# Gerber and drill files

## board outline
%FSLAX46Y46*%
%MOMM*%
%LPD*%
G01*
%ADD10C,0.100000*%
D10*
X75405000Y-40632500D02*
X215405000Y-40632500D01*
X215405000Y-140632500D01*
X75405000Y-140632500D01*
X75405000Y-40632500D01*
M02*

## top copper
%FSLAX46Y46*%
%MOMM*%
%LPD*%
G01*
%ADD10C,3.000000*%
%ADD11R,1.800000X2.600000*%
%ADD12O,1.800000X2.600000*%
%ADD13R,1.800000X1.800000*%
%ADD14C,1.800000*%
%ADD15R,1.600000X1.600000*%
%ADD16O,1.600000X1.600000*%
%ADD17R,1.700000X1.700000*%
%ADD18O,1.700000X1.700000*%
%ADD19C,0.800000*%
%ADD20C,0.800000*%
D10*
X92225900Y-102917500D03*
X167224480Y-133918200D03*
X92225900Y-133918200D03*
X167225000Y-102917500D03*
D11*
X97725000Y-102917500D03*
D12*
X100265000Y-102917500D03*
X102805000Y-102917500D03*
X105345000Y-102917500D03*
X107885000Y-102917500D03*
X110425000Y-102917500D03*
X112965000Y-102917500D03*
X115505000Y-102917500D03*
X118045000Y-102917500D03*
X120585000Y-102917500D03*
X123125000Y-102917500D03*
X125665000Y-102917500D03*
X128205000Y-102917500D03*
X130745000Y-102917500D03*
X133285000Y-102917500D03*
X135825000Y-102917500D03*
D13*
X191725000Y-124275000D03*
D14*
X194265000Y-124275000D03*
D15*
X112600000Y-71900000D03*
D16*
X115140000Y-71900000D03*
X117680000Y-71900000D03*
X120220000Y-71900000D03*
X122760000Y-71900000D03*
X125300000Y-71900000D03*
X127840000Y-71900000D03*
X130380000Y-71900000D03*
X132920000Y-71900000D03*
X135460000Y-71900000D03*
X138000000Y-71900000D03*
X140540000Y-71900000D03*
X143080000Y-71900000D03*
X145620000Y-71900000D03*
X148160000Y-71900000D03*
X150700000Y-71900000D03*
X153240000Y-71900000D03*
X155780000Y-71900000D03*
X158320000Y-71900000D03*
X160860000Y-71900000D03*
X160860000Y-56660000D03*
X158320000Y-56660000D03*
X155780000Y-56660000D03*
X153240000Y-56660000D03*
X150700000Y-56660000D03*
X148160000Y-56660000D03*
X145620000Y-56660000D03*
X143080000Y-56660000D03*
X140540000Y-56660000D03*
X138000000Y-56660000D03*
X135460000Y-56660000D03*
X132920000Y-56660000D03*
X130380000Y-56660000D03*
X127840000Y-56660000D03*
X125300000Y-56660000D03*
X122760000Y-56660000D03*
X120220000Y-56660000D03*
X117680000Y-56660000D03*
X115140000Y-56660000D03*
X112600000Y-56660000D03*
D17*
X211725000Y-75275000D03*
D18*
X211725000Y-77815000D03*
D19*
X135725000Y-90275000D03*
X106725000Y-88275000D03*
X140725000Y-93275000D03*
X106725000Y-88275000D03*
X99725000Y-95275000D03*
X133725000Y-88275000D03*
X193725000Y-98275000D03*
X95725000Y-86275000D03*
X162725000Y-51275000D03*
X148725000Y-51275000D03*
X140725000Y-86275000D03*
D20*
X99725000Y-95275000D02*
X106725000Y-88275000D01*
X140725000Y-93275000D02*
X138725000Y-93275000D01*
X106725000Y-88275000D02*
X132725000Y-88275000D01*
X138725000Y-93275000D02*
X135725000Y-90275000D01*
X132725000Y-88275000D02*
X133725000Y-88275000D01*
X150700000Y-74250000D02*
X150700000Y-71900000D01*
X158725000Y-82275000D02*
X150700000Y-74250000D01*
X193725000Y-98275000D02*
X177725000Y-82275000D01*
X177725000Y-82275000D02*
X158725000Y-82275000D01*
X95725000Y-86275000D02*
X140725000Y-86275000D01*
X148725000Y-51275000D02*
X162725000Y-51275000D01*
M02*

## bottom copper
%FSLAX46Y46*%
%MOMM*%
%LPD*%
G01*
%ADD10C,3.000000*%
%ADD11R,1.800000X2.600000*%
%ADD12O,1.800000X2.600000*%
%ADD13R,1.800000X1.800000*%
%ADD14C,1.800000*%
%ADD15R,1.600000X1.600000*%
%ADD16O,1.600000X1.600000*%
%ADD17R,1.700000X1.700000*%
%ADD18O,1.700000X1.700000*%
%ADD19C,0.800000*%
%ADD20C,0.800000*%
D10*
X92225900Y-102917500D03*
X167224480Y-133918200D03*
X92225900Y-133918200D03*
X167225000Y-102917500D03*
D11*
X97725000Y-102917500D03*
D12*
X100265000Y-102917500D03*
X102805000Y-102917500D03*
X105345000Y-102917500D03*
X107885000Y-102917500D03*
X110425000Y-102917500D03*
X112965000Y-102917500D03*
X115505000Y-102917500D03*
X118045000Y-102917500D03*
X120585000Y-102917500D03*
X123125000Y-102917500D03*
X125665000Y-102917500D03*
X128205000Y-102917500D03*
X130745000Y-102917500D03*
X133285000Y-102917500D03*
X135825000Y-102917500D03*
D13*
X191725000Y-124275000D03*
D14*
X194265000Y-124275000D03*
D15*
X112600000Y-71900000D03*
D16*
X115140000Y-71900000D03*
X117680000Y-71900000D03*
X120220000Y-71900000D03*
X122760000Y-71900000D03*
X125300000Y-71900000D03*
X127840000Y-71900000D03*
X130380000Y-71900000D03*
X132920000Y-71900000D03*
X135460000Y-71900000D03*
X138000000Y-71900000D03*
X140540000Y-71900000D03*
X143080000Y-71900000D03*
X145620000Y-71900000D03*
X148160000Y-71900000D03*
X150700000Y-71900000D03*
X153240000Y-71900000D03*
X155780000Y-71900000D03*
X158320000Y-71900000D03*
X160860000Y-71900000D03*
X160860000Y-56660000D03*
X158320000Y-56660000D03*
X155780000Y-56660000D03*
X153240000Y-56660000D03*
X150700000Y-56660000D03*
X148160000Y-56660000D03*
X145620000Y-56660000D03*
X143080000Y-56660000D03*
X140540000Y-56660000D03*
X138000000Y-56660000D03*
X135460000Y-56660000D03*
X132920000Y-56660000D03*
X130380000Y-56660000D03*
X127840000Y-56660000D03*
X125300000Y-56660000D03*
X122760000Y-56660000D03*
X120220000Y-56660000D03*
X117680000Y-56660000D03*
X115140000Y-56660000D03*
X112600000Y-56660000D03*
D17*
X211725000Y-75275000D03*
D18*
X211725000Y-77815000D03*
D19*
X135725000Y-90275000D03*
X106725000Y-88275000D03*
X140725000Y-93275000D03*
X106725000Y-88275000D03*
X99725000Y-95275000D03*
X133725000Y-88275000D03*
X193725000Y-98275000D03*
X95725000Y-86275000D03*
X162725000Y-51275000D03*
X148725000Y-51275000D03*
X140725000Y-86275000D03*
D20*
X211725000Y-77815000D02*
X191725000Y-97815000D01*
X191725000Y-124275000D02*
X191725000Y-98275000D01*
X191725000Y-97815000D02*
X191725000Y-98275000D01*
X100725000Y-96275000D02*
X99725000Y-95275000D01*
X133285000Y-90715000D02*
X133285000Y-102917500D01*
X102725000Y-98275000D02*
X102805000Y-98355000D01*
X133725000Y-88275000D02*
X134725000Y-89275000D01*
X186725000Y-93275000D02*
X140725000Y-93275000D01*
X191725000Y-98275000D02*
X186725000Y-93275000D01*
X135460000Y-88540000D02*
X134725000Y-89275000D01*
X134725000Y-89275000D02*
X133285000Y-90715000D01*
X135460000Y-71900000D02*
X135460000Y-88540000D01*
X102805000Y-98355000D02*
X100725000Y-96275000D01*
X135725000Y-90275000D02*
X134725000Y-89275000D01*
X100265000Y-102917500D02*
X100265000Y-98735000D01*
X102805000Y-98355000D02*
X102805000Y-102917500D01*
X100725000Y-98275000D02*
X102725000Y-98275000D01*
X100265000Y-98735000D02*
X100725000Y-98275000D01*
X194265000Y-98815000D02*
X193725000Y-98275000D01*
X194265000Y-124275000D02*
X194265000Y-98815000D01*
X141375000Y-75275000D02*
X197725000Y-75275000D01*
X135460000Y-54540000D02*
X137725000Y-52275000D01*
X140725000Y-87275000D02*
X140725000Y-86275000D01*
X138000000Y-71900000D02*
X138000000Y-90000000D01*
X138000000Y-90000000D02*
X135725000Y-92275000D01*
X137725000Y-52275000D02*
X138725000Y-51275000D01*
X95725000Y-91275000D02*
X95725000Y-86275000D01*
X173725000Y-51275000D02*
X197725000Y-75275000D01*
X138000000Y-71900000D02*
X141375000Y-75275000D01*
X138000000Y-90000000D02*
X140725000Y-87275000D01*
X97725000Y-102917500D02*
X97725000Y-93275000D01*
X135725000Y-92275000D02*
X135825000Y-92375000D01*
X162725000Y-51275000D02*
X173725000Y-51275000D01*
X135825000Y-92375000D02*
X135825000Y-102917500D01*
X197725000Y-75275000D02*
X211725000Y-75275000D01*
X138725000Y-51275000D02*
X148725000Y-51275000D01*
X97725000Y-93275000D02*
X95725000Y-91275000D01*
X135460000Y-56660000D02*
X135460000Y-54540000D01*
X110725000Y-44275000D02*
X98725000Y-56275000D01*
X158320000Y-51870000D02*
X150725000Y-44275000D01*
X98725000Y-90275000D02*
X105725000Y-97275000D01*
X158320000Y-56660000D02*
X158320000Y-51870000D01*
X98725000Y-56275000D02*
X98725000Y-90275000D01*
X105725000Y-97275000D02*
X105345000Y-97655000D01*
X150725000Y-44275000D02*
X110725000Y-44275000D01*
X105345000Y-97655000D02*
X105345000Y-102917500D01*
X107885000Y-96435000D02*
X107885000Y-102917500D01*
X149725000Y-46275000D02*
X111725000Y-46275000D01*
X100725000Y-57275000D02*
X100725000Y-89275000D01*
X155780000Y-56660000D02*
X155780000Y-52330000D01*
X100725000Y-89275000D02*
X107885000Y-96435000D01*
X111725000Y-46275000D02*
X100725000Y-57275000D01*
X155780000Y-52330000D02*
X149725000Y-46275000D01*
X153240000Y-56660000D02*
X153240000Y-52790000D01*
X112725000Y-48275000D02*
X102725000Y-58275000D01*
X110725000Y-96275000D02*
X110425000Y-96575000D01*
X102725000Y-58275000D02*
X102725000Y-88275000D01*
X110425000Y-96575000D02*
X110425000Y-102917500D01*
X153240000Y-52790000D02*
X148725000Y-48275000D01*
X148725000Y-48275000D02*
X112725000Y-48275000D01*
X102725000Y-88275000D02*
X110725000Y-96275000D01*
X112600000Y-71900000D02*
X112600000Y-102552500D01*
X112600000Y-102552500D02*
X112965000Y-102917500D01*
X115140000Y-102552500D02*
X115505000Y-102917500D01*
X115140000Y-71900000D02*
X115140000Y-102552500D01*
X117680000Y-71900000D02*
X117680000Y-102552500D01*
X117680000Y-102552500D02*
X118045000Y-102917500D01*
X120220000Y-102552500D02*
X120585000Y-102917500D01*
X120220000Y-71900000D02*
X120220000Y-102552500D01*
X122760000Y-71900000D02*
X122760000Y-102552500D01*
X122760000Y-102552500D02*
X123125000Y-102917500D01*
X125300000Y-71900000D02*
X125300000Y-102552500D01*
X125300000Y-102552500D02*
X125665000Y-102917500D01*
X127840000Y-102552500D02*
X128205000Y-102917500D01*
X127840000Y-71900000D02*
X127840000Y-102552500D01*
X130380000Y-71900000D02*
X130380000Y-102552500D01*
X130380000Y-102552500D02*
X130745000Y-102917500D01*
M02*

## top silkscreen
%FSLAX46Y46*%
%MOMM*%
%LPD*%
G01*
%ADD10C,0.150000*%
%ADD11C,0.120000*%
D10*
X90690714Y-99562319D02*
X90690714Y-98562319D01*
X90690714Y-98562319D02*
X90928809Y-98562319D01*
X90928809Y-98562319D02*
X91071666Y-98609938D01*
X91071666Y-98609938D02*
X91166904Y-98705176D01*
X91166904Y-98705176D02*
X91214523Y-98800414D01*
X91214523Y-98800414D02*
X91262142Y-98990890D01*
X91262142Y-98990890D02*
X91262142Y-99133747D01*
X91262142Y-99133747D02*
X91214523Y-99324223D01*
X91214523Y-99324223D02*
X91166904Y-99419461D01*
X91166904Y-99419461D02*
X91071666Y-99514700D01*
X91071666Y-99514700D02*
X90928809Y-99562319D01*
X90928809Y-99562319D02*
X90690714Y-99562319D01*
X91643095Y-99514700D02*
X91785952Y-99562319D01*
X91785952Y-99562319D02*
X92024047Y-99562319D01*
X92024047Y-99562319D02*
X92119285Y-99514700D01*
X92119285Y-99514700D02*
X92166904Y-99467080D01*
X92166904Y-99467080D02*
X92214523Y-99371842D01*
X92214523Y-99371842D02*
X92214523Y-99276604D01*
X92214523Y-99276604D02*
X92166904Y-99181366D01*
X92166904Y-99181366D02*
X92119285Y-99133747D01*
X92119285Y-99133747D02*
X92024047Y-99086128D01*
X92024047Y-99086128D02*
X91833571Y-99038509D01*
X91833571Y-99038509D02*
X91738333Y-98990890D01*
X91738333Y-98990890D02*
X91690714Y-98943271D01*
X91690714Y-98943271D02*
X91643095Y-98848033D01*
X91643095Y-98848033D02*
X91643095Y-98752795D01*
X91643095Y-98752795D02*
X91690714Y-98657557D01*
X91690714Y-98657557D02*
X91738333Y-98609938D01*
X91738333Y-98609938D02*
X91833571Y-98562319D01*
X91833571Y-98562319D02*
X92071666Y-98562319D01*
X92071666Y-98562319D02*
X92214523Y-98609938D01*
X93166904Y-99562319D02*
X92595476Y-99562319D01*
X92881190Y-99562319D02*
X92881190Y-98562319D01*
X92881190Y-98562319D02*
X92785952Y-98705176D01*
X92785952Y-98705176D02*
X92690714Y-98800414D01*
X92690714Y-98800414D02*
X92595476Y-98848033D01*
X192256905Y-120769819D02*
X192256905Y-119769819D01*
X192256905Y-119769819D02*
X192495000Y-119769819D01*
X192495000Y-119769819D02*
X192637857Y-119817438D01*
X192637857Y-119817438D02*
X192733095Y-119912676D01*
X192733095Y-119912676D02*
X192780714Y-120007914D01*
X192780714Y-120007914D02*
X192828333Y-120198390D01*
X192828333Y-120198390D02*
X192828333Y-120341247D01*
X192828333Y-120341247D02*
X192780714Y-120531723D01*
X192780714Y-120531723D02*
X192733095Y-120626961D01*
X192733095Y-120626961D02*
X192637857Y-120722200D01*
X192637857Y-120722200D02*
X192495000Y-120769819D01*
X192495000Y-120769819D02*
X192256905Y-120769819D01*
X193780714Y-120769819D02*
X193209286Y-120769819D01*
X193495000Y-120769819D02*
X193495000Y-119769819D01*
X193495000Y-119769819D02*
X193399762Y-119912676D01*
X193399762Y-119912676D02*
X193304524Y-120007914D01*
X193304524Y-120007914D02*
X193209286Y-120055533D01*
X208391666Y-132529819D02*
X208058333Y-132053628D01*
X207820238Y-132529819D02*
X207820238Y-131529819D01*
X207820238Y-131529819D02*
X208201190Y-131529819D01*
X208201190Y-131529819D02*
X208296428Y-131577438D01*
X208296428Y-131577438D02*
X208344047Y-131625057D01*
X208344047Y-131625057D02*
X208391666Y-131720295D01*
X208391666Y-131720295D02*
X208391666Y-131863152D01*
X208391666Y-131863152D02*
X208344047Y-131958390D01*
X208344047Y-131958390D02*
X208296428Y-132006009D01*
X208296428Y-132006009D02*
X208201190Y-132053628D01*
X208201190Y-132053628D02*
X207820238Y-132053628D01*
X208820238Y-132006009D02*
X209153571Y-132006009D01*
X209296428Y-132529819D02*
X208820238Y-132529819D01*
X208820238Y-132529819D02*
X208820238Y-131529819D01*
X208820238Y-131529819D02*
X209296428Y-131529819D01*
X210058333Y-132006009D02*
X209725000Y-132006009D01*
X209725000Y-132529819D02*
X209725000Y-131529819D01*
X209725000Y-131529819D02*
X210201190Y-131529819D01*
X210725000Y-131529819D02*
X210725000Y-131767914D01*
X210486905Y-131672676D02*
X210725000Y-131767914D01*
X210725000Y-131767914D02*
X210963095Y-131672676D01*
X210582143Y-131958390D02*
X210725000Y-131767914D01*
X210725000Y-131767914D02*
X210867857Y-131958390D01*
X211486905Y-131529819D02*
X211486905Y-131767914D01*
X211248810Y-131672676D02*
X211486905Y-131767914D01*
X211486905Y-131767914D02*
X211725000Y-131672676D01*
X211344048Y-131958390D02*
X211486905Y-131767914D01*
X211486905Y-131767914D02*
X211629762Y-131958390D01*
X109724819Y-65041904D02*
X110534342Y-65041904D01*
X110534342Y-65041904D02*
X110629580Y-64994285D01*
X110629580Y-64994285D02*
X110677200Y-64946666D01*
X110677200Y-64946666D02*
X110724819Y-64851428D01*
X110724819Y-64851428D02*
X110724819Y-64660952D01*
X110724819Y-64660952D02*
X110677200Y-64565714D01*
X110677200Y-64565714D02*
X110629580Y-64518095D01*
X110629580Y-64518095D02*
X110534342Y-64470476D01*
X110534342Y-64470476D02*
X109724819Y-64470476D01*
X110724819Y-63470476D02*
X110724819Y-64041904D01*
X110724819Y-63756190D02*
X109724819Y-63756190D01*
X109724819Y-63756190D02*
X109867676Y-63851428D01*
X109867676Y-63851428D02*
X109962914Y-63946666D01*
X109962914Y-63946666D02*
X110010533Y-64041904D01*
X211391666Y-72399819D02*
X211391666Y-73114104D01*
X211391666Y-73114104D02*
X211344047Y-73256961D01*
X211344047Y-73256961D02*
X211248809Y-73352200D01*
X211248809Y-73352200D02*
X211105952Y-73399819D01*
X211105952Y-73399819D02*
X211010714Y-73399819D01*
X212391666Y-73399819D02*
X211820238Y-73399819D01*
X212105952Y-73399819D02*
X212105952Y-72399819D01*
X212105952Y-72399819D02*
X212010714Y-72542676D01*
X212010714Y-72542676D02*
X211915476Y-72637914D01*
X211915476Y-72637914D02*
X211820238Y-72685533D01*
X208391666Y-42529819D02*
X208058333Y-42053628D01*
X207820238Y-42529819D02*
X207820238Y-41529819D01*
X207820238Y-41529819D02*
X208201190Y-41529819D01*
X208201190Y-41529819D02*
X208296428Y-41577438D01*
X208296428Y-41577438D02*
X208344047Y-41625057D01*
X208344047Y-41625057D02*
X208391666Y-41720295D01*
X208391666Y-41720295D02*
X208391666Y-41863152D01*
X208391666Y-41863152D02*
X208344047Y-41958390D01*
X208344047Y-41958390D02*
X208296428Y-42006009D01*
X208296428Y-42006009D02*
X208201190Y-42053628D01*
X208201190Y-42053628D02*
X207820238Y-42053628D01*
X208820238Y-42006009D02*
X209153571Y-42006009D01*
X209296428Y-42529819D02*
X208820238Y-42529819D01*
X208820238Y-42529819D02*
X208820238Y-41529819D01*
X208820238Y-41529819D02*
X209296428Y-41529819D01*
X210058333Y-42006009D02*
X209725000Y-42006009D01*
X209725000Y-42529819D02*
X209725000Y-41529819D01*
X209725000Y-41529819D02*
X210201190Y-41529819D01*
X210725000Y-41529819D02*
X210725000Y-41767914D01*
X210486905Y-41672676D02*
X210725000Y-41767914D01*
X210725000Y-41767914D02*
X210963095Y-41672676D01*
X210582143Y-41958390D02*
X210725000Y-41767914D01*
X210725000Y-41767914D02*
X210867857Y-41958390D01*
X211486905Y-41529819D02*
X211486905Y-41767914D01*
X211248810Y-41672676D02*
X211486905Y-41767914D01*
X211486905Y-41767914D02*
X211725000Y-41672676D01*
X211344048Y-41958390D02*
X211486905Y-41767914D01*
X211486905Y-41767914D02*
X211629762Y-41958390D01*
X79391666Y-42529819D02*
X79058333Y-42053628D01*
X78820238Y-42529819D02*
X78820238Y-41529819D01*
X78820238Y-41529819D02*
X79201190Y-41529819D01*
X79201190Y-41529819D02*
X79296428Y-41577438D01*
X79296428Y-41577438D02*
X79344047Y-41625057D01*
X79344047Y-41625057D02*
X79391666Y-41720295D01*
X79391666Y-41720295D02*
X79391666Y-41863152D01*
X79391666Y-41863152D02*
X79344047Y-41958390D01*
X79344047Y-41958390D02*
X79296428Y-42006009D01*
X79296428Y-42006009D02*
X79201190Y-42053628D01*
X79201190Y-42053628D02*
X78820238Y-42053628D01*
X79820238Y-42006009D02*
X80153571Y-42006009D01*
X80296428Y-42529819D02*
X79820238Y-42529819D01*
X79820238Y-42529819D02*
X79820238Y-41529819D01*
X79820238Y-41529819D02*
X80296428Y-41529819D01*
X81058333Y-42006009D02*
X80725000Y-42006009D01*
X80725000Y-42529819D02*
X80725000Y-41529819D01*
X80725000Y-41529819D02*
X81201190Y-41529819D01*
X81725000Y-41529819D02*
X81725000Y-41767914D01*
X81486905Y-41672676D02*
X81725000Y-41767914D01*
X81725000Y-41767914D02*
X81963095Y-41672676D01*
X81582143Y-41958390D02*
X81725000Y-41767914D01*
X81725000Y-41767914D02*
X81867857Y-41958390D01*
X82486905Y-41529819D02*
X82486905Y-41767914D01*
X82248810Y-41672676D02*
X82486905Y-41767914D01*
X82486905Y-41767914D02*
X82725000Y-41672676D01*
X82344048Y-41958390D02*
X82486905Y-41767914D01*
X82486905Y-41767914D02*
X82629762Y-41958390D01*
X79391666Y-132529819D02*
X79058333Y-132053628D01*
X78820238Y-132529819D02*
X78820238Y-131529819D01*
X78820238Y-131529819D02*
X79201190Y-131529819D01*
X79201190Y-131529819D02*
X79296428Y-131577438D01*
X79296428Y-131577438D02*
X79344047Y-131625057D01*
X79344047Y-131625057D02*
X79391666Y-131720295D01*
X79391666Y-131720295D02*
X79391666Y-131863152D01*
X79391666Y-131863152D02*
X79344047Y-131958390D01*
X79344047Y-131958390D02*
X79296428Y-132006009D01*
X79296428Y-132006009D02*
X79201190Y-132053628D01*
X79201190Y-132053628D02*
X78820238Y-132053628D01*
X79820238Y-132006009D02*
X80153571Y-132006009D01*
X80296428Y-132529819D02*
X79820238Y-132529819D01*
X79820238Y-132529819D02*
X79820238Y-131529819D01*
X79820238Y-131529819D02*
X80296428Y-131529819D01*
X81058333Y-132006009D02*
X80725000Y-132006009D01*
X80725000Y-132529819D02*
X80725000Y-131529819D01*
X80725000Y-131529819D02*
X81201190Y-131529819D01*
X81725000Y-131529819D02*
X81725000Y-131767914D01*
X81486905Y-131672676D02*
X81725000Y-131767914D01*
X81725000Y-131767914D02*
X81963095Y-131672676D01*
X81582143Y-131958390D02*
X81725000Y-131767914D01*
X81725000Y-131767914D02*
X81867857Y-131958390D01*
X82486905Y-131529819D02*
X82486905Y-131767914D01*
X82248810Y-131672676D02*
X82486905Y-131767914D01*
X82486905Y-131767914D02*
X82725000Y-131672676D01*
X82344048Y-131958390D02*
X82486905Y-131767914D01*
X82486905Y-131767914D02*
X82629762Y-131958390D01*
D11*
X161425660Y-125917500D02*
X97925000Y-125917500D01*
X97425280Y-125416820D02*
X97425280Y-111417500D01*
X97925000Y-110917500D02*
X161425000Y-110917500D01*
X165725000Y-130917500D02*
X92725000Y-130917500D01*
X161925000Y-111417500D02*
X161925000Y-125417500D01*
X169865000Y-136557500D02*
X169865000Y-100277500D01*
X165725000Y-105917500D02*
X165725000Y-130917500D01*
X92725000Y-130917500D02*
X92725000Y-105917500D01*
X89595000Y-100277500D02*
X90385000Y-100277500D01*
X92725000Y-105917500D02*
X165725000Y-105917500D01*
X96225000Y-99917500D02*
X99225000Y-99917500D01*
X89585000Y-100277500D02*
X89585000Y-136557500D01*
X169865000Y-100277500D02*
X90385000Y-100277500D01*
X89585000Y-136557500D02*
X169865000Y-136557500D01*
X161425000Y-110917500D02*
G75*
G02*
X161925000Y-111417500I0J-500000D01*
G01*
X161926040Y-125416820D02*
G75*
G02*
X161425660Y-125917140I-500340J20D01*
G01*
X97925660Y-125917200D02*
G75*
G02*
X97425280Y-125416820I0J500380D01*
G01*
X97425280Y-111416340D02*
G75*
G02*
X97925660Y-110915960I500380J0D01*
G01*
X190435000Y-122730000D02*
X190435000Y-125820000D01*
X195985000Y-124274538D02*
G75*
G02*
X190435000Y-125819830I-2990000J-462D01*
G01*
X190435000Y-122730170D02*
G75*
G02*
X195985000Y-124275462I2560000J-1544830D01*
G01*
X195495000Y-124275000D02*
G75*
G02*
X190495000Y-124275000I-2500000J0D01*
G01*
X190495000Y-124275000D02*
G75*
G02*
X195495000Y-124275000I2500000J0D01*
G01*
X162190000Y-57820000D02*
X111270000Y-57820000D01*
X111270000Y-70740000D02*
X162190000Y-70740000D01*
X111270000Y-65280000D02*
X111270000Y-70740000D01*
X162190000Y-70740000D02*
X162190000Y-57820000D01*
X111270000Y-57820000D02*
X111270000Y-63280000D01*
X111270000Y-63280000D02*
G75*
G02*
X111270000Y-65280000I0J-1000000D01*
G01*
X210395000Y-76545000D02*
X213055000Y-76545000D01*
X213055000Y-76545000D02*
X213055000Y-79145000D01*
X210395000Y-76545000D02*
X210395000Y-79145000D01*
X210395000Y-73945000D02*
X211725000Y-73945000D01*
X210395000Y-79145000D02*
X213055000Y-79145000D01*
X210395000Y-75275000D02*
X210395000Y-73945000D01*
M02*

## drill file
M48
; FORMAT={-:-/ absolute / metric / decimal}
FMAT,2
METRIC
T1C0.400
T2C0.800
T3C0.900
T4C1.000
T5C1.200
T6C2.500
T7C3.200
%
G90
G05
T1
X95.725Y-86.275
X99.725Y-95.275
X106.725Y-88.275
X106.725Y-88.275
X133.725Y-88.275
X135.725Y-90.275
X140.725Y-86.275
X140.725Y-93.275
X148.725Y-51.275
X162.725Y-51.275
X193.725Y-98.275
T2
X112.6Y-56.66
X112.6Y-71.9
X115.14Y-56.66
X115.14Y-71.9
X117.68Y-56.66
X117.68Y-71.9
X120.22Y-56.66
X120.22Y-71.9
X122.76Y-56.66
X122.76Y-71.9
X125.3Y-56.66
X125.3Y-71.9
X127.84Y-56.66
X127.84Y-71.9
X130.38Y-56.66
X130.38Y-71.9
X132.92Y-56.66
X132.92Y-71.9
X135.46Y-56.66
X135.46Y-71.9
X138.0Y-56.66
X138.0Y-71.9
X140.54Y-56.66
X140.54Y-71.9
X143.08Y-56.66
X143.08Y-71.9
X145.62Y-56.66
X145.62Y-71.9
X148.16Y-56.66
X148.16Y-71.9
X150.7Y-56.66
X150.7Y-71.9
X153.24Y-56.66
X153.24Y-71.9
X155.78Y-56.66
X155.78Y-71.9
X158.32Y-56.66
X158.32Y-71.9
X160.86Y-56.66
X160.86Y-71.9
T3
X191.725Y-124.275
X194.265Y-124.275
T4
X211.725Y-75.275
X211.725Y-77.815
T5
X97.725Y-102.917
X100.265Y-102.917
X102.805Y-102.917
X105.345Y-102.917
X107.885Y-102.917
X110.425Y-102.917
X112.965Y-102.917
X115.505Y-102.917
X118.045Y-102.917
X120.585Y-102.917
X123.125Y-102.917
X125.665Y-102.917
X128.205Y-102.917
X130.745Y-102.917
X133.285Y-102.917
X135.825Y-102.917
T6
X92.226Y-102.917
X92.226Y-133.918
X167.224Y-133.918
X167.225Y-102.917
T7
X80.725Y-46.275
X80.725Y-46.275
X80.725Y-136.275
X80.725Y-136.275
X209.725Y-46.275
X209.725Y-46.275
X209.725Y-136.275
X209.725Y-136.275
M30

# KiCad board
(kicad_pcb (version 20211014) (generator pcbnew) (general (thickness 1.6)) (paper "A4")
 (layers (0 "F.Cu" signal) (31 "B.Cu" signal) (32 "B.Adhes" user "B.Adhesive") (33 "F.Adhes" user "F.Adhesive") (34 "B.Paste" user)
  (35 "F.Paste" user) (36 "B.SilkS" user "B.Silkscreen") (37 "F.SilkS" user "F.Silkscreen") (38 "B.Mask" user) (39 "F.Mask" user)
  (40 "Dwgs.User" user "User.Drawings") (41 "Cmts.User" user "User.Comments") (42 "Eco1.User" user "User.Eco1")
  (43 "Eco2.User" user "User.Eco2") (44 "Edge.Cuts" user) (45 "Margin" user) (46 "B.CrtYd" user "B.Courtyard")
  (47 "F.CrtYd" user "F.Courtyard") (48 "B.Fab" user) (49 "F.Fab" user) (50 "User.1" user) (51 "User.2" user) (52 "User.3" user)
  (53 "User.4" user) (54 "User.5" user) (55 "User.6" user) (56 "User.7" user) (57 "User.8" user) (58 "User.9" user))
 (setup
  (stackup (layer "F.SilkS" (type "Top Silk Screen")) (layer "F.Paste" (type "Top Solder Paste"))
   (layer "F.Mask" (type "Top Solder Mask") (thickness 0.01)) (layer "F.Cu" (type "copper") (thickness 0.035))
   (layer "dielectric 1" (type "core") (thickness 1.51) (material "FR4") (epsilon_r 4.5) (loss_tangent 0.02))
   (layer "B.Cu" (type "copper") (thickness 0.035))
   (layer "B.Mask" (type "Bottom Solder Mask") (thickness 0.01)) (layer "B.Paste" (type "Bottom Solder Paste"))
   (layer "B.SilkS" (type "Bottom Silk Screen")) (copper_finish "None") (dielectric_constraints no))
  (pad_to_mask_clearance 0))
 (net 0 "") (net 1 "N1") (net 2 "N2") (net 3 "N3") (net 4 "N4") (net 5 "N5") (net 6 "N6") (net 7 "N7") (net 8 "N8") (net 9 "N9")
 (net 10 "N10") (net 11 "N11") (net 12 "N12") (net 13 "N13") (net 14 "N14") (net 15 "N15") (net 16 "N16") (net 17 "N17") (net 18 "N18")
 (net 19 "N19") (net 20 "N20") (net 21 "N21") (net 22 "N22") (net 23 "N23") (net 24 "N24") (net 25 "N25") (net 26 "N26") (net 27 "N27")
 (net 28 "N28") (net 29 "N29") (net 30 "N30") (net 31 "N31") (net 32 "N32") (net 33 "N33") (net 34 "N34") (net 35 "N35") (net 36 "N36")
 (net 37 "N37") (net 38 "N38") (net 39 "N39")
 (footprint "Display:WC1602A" (layer "F.Cu") (at 97.725 102.9175)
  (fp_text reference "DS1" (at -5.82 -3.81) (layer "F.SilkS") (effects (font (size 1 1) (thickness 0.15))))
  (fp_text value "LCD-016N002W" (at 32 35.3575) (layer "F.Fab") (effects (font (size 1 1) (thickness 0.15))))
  (fp_line (start 63.70066 23) (end 0.2 23) (layer "F.SilkS") (width 0.12))
  (fp_line (start -0.29972 22.49932) (end -0.29972 8.5) (layer "F.SilkS") (width 0.12))
  (fp_line (start 0.2 8) (end 63.7 8) (layer "F.SilkS") (width 0.12))
  (fp_line (start 68 28) (end -5 28) (layer "F.SilkS") (width 0.12))
  (fp_line (start 64.2 8.5) (end 64.2 22.5) (layer "F.SilkS") (width 0.12))
  (fp_line (start 72.14 33.64) (end 72.14 -2.64) (layer "F.SilkS") (width 0.12))
  (fp_line (start 68 3) (end 68 28) (layer "F.SilkS") (width 0.12))
  (fp_line (start -5 28) (end -5 3) (layer "F.SilkS") (width 0.12))
  (fp_line (start -8.13 -2.64) (end -7.34 -2.64) (layer "F.SilkS") (width 0.12))
  (fp_line (start -5 3) (end 68 3) (layer "F.SilkS") (width 0.12))
  (fp_line (start -1.5 -3) (end 1.5 -3) (layer "F.SilkS") (width 0.12))
  (fp_line (start -8.14 -2.64) (end -8.14 33.64) (layer "F.SilkS") (width 0.12))
  (fp_line (start 72.14 -2.64) (end -7.34 -2.64) (layer "F.SilkS") (width 0.12))
  (fp_line (start -8.14 33.64) (end 72.14 33.64) (layer "F.SilkS") (width 0.12))
  (fp_arc (start 63.7 8) (mid 64.053553 8.146447) (end 64.2 8.5) (layer "F.SilkS") (width 0.12))
  (fp_arc (start 64.20104 22.49932) (mid 64.054479 22.85315) (end 63.70066 22.9997) (layer "F.SilkS") (width 0.12))
  (fp_arc (start 0.20066 22.9997) (mid -0.153162 22.853142) (end -0.29972 22.49932) (layer "F.SilkS") (width 0.12))
  (fp_arc (start -0.29972 8.49884) (mid -0.153162 8.145018) (end 0.20066 7.99846) (layer "F.SilkS") (width 0.12))
  (pad "" thru_hole circle (at -5.4991 0) (size 3 3) (drill 2.5) (layers *.Cu *.Mask))
  (pad "" thru_hole circle (at 69.49948 31.0007) (size 3 3) (drill 2.5) (layers *.Cu *.Mask))
  (pad "" thru_hole circle (at -5.4991 31.0007) (size 3 3) (drill 2.5) (layers *.Cu *.Mask))
  (pad "" thru_hole circle (at 69.5 0) (size 3 3) (drill 2.5) (layers *.Cu *.Mask))
  (pad "1" thru_hole rect (at 0 0) (size 1.8 2.6) (drill 1.2) (layers *.Cu *.Mask) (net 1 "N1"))
  (pad "2" thru_hole oval (at 2.54 0) (size 1.8 2.6) (drill 1.2) (layers *.Cu *.Mask) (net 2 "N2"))
  (pad "3" thru_hole oval (at 5.08 0) (size 1.8 2.6) (drill 1.2) (layers *.Cu *.Mask) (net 2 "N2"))
  (pad "4" thru_hole oval (at 7.62 0) (size 1.8 2.6) (drill 1.2) (layers *.Cu *.Mask) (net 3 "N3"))
  (pad "5" thru_hole oval (at 10.16 0) (size 1.8 2.6) (drill 1.2) (layers *.Cu *.Mask) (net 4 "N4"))
  (pad "6" thru_hole oval (at 12.7 0) (size 1.8 2.6) (drill 1.2) (layers *.Cu *.Mask) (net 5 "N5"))
  (pad "7" thru_hole oval (at 15.24 0) (size 1.8 2.6) (drill 1.2) (layers *.Cu *.Mask) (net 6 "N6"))
  (pad "8" thru_hole oval (at 17.78 0) (size 1.8 2.6) (drill 1.2) (layers *.Cu *.Mask) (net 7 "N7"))
  (pad "9" thru_hole oval (at 20.32 0) (size 1.8 2.6) (drill 1.2) (layers *.Cu *.Mask) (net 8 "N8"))
  (pad "10" thru_hole oval (at 22.86 0) (size 1.8 2.6) (drill 1.2) (layers *.Cu *.Mask) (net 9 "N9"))
  (pad "11" thru_hole oval (at 25.4 0) (size 1.8 2.6) (drill 1.2) (layers *.Cu *.Mask) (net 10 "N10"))
  (pad "12" thru_hole oval (at 27.94 0) (size 1.8 2.6) (drill 1.2) (layers *.Cu *.Mask) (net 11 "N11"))
  (pad "13" thru_hole oval (at 30.48 0) (size 1.8 2.6) (drill 1.2) (layers *.Cu *.Mask) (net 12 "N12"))
  (pad "14" thru_hole oval (at 33.02 0) (size 1.8 2.6) (drill 1.2) (layers *.Cu *.Mask) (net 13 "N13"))
  (pad "15" thru_hole oval (at 35.56 0) (size 1.8 2.6) (drill 1.2) (layers *.Cu *.Mask) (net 2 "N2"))
  (pad "16" thru_hole oval (at 38.1 0) (size 1.8 2.6) (drill 1.2) (layers *.Cu *.Mask) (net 1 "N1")))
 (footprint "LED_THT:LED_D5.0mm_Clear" (layer "F.Cu") (at 191.725 124.275)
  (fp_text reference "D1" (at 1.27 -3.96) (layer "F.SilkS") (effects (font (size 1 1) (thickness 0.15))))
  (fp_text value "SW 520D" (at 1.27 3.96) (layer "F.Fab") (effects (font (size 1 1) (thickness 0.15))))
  (fp_line (start -1.29 -1.545) (end -1.29 1.545) (layer "F.SilkS") (width 0.12))
  (fp_arc (start 4.26 -0.000462) (mid 2.072002 2.880433) (end -1.29 1.54483) (layer "F.SilkS") (width 0.12))
  (fp_arc (start -1.29 -1.54483) (mid 2.072002 -2.880433) (end 4.26 0.000462) (layer "F.SilkS") (width 0.12))
  (fp_circle (center 1.27 0) (end 3.77 0) (layer "F.SilkS") (width 0.12) (fill none))
  (pad "1" thru_hole rect (at 0 0) (size 1.8 1.8) (drill 0.9) (layers *.Cu *.Mask) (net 2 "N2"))
  (pad "2" thru_hole circle (at 2.54 0) (size 1.8 1.8) (drill 0.9) (layers *.Cu *.Mask) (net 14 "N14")))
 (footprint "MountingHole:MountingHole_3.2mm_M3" (layer "F.Cu") (at 209.725 136.275)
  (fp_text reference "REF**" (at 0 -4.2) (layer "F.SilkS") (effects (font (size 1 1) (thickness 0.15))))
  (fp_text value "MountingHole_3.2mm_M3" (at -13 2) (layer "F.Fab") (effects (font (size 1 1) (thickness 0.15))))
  (pad "" np_thru_hole circle (at 0 0) (size 3.2 3.2) (drill 3.2) (layers *.Cu *.Mask))
  (pad "" np_thru_hole circle (at 0 0) (size 3.2 3.2) (drill 3.2) (layers *.Cu *.Mask)))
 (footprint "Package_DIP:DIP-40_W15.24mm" (layer "F.Cu") (at 112.6 71.9 90)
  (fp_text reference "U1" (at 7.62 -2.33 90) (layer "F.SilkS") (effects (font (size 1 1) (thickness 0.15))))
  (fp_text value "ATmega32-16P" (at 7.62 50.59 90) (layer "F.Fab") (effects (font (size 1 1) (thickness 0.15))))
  (fp_line (start 14.08 49.59) (end 14.08 -1.33) (layer "F.SilkS") (width 0.12))
  (fp_line (start 1.16 -1.33) (end 1.16 49.59) (layer "F.SilkS") (width 0.12))
  (fp_line (start 6.62 -1.33) (end 1.16 -1.33) (layer "F.SilkS") (width 0.12))
  (fp_line (start 1.16 49.59) (end 14.08 49.59) (layer "F.SilkS") (width 0.12))
  (fp_line (start 14.08 -1.33) (end 8.62 -1.33) (layer "F.SilkS") (width 0.12))
  (fp_arc (start 8.62 -1.33) (mid 7.62 -0.33) (end 6.62 -1.33) (layer "F.SilkS") (width 0.12))
  (pad "1" thru_hole rect (at 0 0 90) (size 1.6 1.6) (drill 0.8) (layers *.Cu *.Mask) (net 6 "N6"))
  (pad "2" thru_hole oval (at 0 2.54 90) (size 1.6 1.6) (drill 0.8) (layers *.Cu *.Mask) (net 7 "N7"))
  (pad "3" thru_hole oval (at 0 5.08 90) (size 1.6 1.6) (drill 0.8) (layers *.Cu *.Mask) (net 8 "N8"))
  (pad "4" thru_hole oval (at 0 7.62 90) (size 1.6 1.6) (drill 0.8) (layers *.Cu *.Mask) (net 9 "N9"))
  (pad "5" thru_hole oval (at 0 10.16 90) (size 1.6 1.6) (drill 0.8) (layers *.Cu *.Mask) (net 10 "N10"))
  (pad "6" thru_hole oval (at 0 12.7 90) (size 1.6 1.6) (drill 0.8) (layers *.Cu *.Mask) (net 11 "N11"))
  (pad "7" thru_hole oval (at 0 15.24 90) (size 1.6 1.6) (drill 0.8) (layers *.Cu *.Mask) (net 12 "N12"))
  (pad "8" thru_hole oval (at 0 17.78 90) (size 1.6 1.6) (drill 0.8) (layers *.Cu *.Mask) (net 13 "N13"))
  (pad "9" thru_hole oval (at 0 20.32 90) (size 1.6 1.6) (drill 0.8) (layers *.Cu *.Mask) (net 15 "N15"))
  (pad "10" thru_hole oval (at 0 22.86 90) (size 1.6 1.6) (drill 0.8) (layers *.Cu *.Mask) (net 2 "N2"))
  (pad "11" thru_hole oval (at 0 25.4 90) (size 1.6 1.6) (drill 0.8) (layers *.Cu *.Mask) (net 1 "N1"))
  (pad "12" thru_hole oval (at 0 27.94 90) (size 1.6 1.6) (drill 0.8) (layers *.Cu *.Mask) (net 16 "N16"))
  (pad "13" thru_hole oval (at 0 30.48 90) (size 1.6 1.6) (drill 0.8) (layers *.Cu *.Mask) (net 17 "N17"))
  (pad "14" thru_hole oval (at 0 33.02 90) (size 1.6 1.6) (drill 0.8) (layers *.Cu *.Mask) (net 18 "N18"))
  (pad "15" thru_hole oval (at 0 35.56 90) (size 1.6 1.6) (drill 0.8) (layers *.Cu *.Mask) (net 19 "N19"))
  (pad "16" thru_hole oval (at 0 38.1 90) (size 1.6 1.6) (drill 0.8) (layers *.Cu *.Mask) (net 14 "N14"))
  (pad "17" thru_hole oval (at 0 40.64 90) (size 1.6 1.6) (drill 0.8) (layers *.Cu *.Mask) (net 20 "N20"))
  (pad "18" thru_hole oval (at 0 43.18 90) (size 1.6 1.6) (drill 0.8) (layers *.Cu *.Mask) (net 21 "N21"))
  (pad "19" thru_hole oval (at 0 45.72 90) (size 1.6 1.6) (drill 0.8) (layers *.Cu *.Mask) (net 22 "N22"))
  (pad "20" thru_hole oval (at 0 48.26 90) (size 1.6 1.6) (drill 0.8) (layers *.Cu *.Mask) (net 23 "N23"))
  (pad "21" thru_hole oval (at 15.24 48.26 90) (size 1.6 1.6) (drill 0.8) (layers *.Cu *.Mask) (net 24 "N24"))
  (pad "22" thru_hole oval (at 15.24 45.72 90) (size 1.6 1.6) (drill 0.8) (layers *.Cu *.Mask) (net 3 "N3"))
  (pad "23" thru_hole oval (at 15.24 43.18 90) (size 1.6 1.6) (drill 0.8) (layers *.Cu *.Mask) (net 4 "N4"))
  (pad "24" thru_hole oval (at 15.24 40.64 90) (size 1.6 1.6) (drill 0.8) (layers *.Cu *.Mask) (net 5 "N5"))
  (pad "25" thru_hole oval (at 15.24 38.1 90) (size 1.6 1.6) (drill 0.8) (layers *.Cu *.Mask) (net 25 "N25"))
  (pad "26" thru_hole oval (at 15.24 35.56 90) (size 1.6 1.6) (drill 0.8) (layers *.Cu *.Mask) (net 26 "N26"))
  (pad "27" thru_hole oval (at 15.24 33.02 90) (size 1.6 1.6) (drill 0.8) (layers *.Cu *.Mask) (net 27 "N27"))
  (pad "28" thru_hole oval (at 15.24 30.48 90) (size 1.6 1.6) (drill 0.8) (layers *.Cu *.Mask) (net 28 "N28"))
  (pad "29" thru_hole oval (at 15.24 27.94 90) (size 1.6 1.6) (drill 0.8) (layers *.Cu *.Mask) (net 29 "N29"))
  (pad "30" thru_hole oval (at 15.24 25.4 90) (size 1.6 1.6) (drill 0.8) (layers *.Cu *.Mask) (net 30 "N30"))
  (pad "31" thru_hole oval (at 15.24 22.86 90) (size 1.6 1.6) (drill 0.8) (layers *.Cu *.Mask) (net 1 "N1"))
  (pad "32" thru_hole oval (at 15.24 20.32 90) (size 1.6 1.6) (drill 0.8) (layers *.Cu *.Mask) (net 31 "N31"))
  (pad "33" thru_hole oval (at 15.24 17.78 90) (size 1.6 1.6) (drill 0.8) (layers *.Cu *.Mask) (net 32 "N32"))
  (pad "34" thru_hole oval (at 15.24 15.24 90) (size 1.6 1.6) (drill 0.8) (layers *.Cu *.Mask) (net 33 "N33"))
  (pad "35" thru_hole oval (at 15.24 12.7 90) (size 1.6 1.6) (drill 0.8) (layers *.Cu *.Mask) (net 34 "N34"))
  (pad "36" thru_hole oval (at 15.24 10.16 90) (size 1.6 1.6) (drill 0.8) (layers *.Cu *.Mask) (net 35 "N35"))
  (pad "37" thru_hole oval (at 15.24 7.62 90) (size 1.6 1.6) (drill 0.8) (layers *.Cu *.Mask) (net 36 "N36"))
  (pad "38" thru_hole oval (at 15.24 5.08 90) (size 1.6 1.6) (drill 0.8) (layers *.Cu *.Mask) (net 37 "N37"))
  (pad "39" thru_hole oval (at 15.24 2.54 90) (size 1.6 1.6) (drill 0.8) (layers *.Cu *.Mask) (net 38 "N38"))
  (pad "40" thru_hole oval (at 15.24 0 90) (size 1.6 1.6) (drill 0.8) (layers *.Cu *.Mask) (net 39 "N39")))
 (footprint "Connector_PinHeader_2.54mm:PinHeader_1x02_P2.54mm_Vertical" (layer "F.Cu") (at 211.725 75.275)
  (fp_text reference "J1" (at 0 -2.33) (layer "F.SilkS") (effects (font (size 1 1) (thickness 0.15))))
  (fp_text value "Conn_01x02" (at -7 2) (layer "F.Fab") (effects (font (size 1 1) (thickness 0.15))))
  (fp_line (start -1.33 1.27) (end 1.33 1.27) (layer "F.SilkS") (width 0.12))
  (fp_line (start 1.33 1.27) (end 1.33 3.87) (layer "F.SilkS") (width 0.12))
  (fp_line (start -1.33 1.27) (end -1.33 3.87) (layer "F.SilkS") (width 0.12))
  (fp_line (start -1.33 -1.33) (end 0 -1.33) (layer "F.SilkS") (width 0.12))
  (fp_line (start -1.33 3.87) (end 1.33 3.87) (layer "F.SilkS") (width 0.12))
  (fp_line (start -1.33 0) (end -1.33 -1.33) (layer "F.SilkS") (width 0.12))
  (pad "1" thru_hole rect (at 0 0) (size 1.7 1.7) (drill 1) (layers *.Cu *.Mask) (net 1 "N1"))
  (pad "2" thru_hole oval (at 0 2.54) (size 1.7 1.7) (drill 1) (layers *.Cu *.Mask) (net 2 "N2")))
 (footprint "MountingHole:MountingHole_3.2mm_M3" (layer "F.Cu") (at 209.725 46.275)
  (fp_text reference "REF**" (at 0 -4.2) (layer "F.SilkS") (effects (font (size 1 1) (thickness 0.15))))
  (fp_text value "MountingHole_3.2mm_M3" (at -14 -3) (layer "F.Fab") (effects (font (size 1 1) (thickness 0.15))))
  (pad "" np_thru_hole circle (at 0 0) (size 3.2 3.2) (drill 3.2) (layers *.Cu *.Mask))
  (pad "" np_thru_hole circle (at 0 0) (size 3.2 3.2) (drill 3.2) (layers *.Cu *.Mask)))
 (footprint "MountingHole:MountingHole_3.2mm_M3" (layer "F.Cu") (at 80.725 46.275)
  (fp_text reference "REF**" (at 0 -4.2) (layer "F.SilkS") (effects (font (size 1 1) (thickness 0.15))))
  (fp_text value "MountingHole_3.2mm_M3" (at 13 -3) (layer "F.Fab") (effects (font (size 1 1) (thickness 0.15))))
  (pad "" np_thru_hole circle (at 0 0) (size 3.2 3.2) (drill 3.2) (layers *.Cu *.Mask))
  (pad "" np_thru_hole circle (at 0 0) (size 3.2 3.2) (drill 3.2) (layers *.Cu *.Mask)))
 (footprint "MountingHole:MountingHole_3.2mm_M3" (layer "F.Cu") (at 80.725 136.275)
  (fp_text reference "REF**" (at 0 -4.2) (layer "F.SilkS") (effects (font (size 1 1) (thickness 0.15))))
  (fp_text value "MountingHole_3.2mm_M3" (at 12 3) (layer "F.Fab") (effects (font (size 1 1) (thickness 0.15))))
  (pad "" np_thru_hole circle (at 0 0) (size 3.2 3.2) (drill 3.2) (layers *.Cu *.Mask))
  (pad "" np_thru_hole circle (at 0 0) (size 3.2 3.2) (drill 3.2) (layers *.Cu *.Mask)))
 (gr_rect (start 75.405 40.6325) (end 215.405 140.6325) (layer "Edge.Cuts") (width 0.1) (fill none))
 (segment (start 99.725 95.275) (end 106.725 88.275) (width 0.8) (layer "F.Cu") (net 2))
 (segment (start 140.725 93.275) (end 138.725 93.275) (width 0.8) (layer "F.Cu") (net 2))
 (segment (start 106.725 88.275) (end 132.725 88.275) (width 0.8) (layer "F.Cu") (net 2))
 (segment (start 138.725 93.275) (end 135.725 90.275) (width 0.8) (layer "F.Cu") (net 2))
 (segment (start 132.725 88.275) (end 133.725 88.275) (width 0.8) (layer "F.Cu") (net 2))
 (via (at 135.725 90.275) (size 0.8) (drill 0.4) (layers "F.Cu" "B.Cu") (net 2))
 (via (at 106.725 88.275) (size 0.8) (drill 0.4) (layers "F.Cu" "B.Cu") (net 2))
 (via (at 140.725 93.275) (size 0.8) (drill 0.4) (layers "F.Cu" "B.Cu") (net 2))
 (via (at 106.725 88.275) (size 0.8) (drill 0.4) (layers "F.Cu" "B.Cu") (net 2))
 (via (at 99.725 95.275) (size 0.8) (drill 0.4) (layers "F.Cu" "B.Cu") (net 2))
 (via (at 133.725 88.275) (size 0.8) (drill 0.4) (layers "F.Cu" "B.Cu") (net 2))
 (segment (start 211.725 77.815) (end 191.725 97.815) (width 0.8) (layer "B.Cu") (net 2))
 (segment (start 191.725 124.275) (end 191.725 98.275) (width 0.8) (layer "B.Cu") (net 2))
 (segment (start 191.725 97.815) (end 191.725 98.275) (width 0.8) (layer "B.Cu") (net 2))
 (segment (start 100.725 96.275) (end 99.725 95.275) (width 0.8) (layer "B.Cu") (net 2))
 (segment (start 133.285 90.715) (end 133.285 102.9175) (width 0.8) (layer "B.Cu") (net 2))
 (segment (start 102.725 98.275) (end 102.805 98.355) (width 0.8) (layer "B.Cu") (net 2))
 (segment (start 133.725 88.275) (end 134.725 89.275) (width 0.8) (layer "B.Cu") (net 2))
 (segment (start 186.725 93.275) (end 140.725 93.275) (width 0.8) (layer "B.Cu") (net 2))
 (segment (start 191.725 98.275) (end 186.725 93.275) (width 0.8) (layer "B.Cu") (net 2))
 (segment (start 135.46 88.54) (end 134.725 89.275) (width 0.8) (layer "B.Cu") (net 2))
 (segment (start 134.725 89.275) (end 133.285 90.715) (width 0.8) (layer "B.Cu") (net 2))
 (segment (start 135.46 71.9) (end 135.46 88.54) (width 0.8) (layer "B.Cu") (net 2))
 (segment (start 102.805 98.355) (end 100.725 96.275) (width 0.8) (layer "B.Cu") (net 2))
 (segment (start 135.725 90.275) (end 134.725 89.275) (width 0.8) (layer "B.Cu") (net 2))
 (segment (start 100.265 102.9175) (end 100.265 98.735) (width 0.8) (layer "B.Cu") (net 2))
 (segment (start 102.805 98.355) (end 102.805 102.9175) (width 0.8) (layer "B.Cu") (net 2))
 (segment (start 100.725 98.275) (end 102.725 98.275) (width 0.8) (layer "B.Cu") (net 2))
 (segment (start 100.265 98.735) (end 100.725 98.275) (width 0.8) (layer "B.Cu") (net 2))
 (segment (start 150.7 74.25) (end 150.7 71.9) (width 0.8) (layer "F.Cu") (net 14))
 (segment (start 158.725 82.275) (end 150.7 74.25) (width 0.8) (layer "F.Cu") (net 14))
 (segment (start 193.725 98.275) (end 177.725 82.275) (width 0.8) (layer "F.Cu") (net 14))
 (segment (start 177.725 82.275) (end 158.725 82.275) (width 0.8) (layer "F.Cu") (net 14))
 (via (at 193.725 98.275) (size 0.8) (drill 0.4) (layers "F.Cu" "B.Cu") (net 14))
 (segment (start 194.265 98.815) (end 193.725 98.275) (width 0.8) (layer "B.Cu") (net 14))
 (segment (start 194.265 124.275) (end 194.265 98.815) (width 0.8) (layer "B.Cu") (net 14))
 (segment (start 95.725 86.275) (end 140.725 86.275) (width 0.8) (layer "F.Cu") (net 1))
 (segment (start 148.725 51.275) (end 162.725 51.275) (width 0.8) (layer "F.Cu") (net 1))
 (via (at 95.725 86.275) (size 0.8) (drill 0.4) (layers "F.Cu" "B.Cu") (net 1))
 (via (at 162.725 51.275) (size 0.8) (drill 0.4) (layers "F.Cu" "B.Cu") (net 1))
 (via (at 148.725 51.275) (size 0.8) (drill 0.4) (layers "F.Cu" "B.Cu") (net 1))
 (via (at 140.725 86.275) (size 0.8) (drill 0.4) (layers "F.Cu" "B.Cu") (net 1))
 (segment (start 141.375 75.275) (end 197.725 75.275) (width 0.8) (layer "B.Cu") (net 1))
 (segment (start 135.46 54.54) (end 137.725 52.275) (width 0.8) (layer "B.Cu") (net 1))
 (segment (start 140.725 87.275) (end 140.725 86.275) (width 0.8) (layer "B.Cu") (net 1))
 (segment (start 138 71.9) (end 138 90) (width 0.8) (layer "B.Cu") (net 1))
 (segment (start 138 90) (end 135.725 92.275) (width 0.8) (layer "B.Cu") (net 1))
 (segment (start 137.725 52.275) (end 138.725 51.275) (width 0.8) (layer "B.Cu") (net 1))
 (segment (start 95.725 91.275) (end 95.725 86.275) (width 0.8) (layer "B.Cu") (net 1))
 (segment (start 173.725 51.275) (end 197.725 75.275) (width 0.8) (layer "B.Cu") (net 1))
 (segment (start 138 71.9) (end 141.375 75.275) (width 0.8) (layer "B.Cu") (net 1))
 (segment (start 138 90) (end 140.725 87.275) (width 0.8) (layer "B.Cu") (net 1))
 (segment (start 97.725 102.9175) (end 97.725 93.275) (width 0.8) (layer "B.Cu") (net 1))
 (segment (start 135.725 92.275) (end 135.825 92.375) (width 0.8) (layer "B.Cu") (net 1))
 (segment (start 162.725 51.275) (end 173.725 51.275) (width 0.8) (layer "B.Cu") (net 1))
 (segment (start 135.825 92.375) (end 135.825 102.9175) (width 0.8) (layer "B.Cu") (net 1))
 (segment (start 197.725 75.275) (end 211.725 75.275) (width 0.8) (layer "B.Cu") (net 1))
 (segment (start 138.725 51.275) (end 148.725 51.275) (width 0.8) (layer "B.Cu") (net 1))
 (segment (start 97.725 93.275) (end 95.725 91.275) (width 0.8) (layer "B.Cu") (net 1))
 (segment (start 135.46 56.66) (end 135.46 54.54) (width 0.8) (layer "B.Cu") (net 1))
 (segment (start 110.725 44.275) (end 98.725 56.275) (width 0.8) (layer "B.Cu") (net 3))
 (segment (start 158.32 51.87) (end 150.725 44.275) (width 0.8) (layer "B.Cu") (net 3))
 (segment (start 98.725 90.275) (end 105.725 97.275) (width 0.8) (layer "B.Cu") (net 3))
 (segment (start 158.32 56.66) (end 158.32 51.87) (width 0.8) (layer "B.Cu") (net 3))
 (segment (start 98.725 56.275) (end 98.725 90.275) (width 0.8) (layer "B.Cu") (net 3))
 (segment (start 105.725 97.275) (end 105.345 97.655) (width 0.8) (layer "B.Cu") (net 3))
 (segment (start 150.725 44.275) (end 110.725 44.275) (width 0.8) (layer "B.Cu") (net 3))
 (segment (start 105.345 97.655) (end 105.345 102.9175) (width 0.8) (layer "B.Cu") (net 3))
 (segment (start 107.885 96.435) (end 107.885 102.9175) (width 0.8) (layer "B.Cu") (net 4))
 (segment (start 149.725 46.275) (end 111.725 46.275) (width 0.8) (layer "B.Cu") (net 4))
 (segment (start 100.725 57.275) (end 100.725 89.275) (width 0.8) (layer "B.Cu") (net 4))
 (segment (start 155.78 56.66) (end 155.78 52.33) (width 0.8) (layer "B.Cu") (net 4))
 (segment (start 100.725 89.275) (end 107.885 96.435) (width 0.8) (layer "B.Cu") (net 4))
 (segment (start 111.725 46.275) (end 100.725 57.275) (width 0.8) (layer "B.Cu") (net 4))
 (segment (start 155.78 52.33) (end 149.725 46.275) (width 0.8) (layer "B.Cu") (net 4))
 (segment (start 153.24 56.66) (end 153.24 52.79) (width 0.8) (layer "B.Cu") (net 5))
 (segment (start 112.725 48.275) (end 102.725 58.275) (width 0.8) (layer "B.Cu") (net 5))
 (segment (start 110.725 96.275) (end 110.425 96.575) (width 0.8) (layer "B.Cu") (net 5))
 (segment (start 102.725 58.275) (end 102.725 88.275) (width 0.8) (layer "B.Cu") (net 5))
 (segment (start 110.425 96.575) (end 110.425 102.9175) (width 0.8) (layer "B.Cu") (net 5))
 (segment (start 153.24 52.79) (end 148.725 48.275) (width 0.8) (layer "B.Cu") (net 5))
 (segment (start 148.725 48.275) (end 112.725 48.275) (width 0.8) (layer "B.Cu") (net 5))
 (segment (start 102.725 88.275) (end 110.725 96.275) (width 0.8) (layer "B.Cu") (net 5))
 (segment (start 112.6 71.9) (end 112.6 102.5525) (width 0.8) (layer "B.Cu") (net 6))
 (segment (start 112.6 102.5525) (end 112.965 102.9175) (width 0.8) (layer "B.Cu") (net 6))
 (segment (start 115.14 102.5525) (end 115.505 102.9175) (width 0.8) (layer "B.Cu") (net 7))
 (segment (start 115.14 71.9) (end 115.14 102.5525) (width 0.8) (layer "B.Cu") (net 7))
 (segment (start 117.68 71.9) (end 117.68 102.5525) (width 0.8) (layer "B.Cu") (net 8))
 (segment (start 117.68 102.5525) (end 118.045 102.9175) (width 0.8) (layer "B.Cu") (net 8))
 (segment (start 120.22 102.5525) (end 120.585 102.9175) (width 0.8) (layer "B.Cu") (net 9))
 (segment (start 120.22 71.9) (end 120.22 102.5525) (width 0.8) (layer "B.Cu") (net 9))
 (segment (start 122.76 71.9) (end 122.76 102.5525) (width 0.8) (layer "B.Cu") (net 10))
 (segment (start 122.76 102.5525) (end 123.125 102.9175) (width 0.8) (layer "B.Cu") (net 10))
 (segment (start 125.3 71.9) (end 125.3 102.5525) (width 0.8) (layer "B.Cu") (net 11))
 (segment (start 125.3 102.5525) (end 125.665 102.9175) (width 0.8) (layer "B.Cu") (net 11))
 (segment (start 127.84 102.5525) (end 128.205 102.9175) (width 0.8) (layer "B.Cu") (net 12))
 (segment (start 127.84 71.9) (end 127.84 102.5525) (width 0.8) (layer "B.Cu") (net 12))
 (segment (start 130.38 71.9) (end 130.38 102.5525) (width 0.8) (layer "B.Cu") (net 13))
 (segment (start 130.38 102.5525) (end 130.745 102.9175) (width 0.8) (layer "B.Cu") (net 13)))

